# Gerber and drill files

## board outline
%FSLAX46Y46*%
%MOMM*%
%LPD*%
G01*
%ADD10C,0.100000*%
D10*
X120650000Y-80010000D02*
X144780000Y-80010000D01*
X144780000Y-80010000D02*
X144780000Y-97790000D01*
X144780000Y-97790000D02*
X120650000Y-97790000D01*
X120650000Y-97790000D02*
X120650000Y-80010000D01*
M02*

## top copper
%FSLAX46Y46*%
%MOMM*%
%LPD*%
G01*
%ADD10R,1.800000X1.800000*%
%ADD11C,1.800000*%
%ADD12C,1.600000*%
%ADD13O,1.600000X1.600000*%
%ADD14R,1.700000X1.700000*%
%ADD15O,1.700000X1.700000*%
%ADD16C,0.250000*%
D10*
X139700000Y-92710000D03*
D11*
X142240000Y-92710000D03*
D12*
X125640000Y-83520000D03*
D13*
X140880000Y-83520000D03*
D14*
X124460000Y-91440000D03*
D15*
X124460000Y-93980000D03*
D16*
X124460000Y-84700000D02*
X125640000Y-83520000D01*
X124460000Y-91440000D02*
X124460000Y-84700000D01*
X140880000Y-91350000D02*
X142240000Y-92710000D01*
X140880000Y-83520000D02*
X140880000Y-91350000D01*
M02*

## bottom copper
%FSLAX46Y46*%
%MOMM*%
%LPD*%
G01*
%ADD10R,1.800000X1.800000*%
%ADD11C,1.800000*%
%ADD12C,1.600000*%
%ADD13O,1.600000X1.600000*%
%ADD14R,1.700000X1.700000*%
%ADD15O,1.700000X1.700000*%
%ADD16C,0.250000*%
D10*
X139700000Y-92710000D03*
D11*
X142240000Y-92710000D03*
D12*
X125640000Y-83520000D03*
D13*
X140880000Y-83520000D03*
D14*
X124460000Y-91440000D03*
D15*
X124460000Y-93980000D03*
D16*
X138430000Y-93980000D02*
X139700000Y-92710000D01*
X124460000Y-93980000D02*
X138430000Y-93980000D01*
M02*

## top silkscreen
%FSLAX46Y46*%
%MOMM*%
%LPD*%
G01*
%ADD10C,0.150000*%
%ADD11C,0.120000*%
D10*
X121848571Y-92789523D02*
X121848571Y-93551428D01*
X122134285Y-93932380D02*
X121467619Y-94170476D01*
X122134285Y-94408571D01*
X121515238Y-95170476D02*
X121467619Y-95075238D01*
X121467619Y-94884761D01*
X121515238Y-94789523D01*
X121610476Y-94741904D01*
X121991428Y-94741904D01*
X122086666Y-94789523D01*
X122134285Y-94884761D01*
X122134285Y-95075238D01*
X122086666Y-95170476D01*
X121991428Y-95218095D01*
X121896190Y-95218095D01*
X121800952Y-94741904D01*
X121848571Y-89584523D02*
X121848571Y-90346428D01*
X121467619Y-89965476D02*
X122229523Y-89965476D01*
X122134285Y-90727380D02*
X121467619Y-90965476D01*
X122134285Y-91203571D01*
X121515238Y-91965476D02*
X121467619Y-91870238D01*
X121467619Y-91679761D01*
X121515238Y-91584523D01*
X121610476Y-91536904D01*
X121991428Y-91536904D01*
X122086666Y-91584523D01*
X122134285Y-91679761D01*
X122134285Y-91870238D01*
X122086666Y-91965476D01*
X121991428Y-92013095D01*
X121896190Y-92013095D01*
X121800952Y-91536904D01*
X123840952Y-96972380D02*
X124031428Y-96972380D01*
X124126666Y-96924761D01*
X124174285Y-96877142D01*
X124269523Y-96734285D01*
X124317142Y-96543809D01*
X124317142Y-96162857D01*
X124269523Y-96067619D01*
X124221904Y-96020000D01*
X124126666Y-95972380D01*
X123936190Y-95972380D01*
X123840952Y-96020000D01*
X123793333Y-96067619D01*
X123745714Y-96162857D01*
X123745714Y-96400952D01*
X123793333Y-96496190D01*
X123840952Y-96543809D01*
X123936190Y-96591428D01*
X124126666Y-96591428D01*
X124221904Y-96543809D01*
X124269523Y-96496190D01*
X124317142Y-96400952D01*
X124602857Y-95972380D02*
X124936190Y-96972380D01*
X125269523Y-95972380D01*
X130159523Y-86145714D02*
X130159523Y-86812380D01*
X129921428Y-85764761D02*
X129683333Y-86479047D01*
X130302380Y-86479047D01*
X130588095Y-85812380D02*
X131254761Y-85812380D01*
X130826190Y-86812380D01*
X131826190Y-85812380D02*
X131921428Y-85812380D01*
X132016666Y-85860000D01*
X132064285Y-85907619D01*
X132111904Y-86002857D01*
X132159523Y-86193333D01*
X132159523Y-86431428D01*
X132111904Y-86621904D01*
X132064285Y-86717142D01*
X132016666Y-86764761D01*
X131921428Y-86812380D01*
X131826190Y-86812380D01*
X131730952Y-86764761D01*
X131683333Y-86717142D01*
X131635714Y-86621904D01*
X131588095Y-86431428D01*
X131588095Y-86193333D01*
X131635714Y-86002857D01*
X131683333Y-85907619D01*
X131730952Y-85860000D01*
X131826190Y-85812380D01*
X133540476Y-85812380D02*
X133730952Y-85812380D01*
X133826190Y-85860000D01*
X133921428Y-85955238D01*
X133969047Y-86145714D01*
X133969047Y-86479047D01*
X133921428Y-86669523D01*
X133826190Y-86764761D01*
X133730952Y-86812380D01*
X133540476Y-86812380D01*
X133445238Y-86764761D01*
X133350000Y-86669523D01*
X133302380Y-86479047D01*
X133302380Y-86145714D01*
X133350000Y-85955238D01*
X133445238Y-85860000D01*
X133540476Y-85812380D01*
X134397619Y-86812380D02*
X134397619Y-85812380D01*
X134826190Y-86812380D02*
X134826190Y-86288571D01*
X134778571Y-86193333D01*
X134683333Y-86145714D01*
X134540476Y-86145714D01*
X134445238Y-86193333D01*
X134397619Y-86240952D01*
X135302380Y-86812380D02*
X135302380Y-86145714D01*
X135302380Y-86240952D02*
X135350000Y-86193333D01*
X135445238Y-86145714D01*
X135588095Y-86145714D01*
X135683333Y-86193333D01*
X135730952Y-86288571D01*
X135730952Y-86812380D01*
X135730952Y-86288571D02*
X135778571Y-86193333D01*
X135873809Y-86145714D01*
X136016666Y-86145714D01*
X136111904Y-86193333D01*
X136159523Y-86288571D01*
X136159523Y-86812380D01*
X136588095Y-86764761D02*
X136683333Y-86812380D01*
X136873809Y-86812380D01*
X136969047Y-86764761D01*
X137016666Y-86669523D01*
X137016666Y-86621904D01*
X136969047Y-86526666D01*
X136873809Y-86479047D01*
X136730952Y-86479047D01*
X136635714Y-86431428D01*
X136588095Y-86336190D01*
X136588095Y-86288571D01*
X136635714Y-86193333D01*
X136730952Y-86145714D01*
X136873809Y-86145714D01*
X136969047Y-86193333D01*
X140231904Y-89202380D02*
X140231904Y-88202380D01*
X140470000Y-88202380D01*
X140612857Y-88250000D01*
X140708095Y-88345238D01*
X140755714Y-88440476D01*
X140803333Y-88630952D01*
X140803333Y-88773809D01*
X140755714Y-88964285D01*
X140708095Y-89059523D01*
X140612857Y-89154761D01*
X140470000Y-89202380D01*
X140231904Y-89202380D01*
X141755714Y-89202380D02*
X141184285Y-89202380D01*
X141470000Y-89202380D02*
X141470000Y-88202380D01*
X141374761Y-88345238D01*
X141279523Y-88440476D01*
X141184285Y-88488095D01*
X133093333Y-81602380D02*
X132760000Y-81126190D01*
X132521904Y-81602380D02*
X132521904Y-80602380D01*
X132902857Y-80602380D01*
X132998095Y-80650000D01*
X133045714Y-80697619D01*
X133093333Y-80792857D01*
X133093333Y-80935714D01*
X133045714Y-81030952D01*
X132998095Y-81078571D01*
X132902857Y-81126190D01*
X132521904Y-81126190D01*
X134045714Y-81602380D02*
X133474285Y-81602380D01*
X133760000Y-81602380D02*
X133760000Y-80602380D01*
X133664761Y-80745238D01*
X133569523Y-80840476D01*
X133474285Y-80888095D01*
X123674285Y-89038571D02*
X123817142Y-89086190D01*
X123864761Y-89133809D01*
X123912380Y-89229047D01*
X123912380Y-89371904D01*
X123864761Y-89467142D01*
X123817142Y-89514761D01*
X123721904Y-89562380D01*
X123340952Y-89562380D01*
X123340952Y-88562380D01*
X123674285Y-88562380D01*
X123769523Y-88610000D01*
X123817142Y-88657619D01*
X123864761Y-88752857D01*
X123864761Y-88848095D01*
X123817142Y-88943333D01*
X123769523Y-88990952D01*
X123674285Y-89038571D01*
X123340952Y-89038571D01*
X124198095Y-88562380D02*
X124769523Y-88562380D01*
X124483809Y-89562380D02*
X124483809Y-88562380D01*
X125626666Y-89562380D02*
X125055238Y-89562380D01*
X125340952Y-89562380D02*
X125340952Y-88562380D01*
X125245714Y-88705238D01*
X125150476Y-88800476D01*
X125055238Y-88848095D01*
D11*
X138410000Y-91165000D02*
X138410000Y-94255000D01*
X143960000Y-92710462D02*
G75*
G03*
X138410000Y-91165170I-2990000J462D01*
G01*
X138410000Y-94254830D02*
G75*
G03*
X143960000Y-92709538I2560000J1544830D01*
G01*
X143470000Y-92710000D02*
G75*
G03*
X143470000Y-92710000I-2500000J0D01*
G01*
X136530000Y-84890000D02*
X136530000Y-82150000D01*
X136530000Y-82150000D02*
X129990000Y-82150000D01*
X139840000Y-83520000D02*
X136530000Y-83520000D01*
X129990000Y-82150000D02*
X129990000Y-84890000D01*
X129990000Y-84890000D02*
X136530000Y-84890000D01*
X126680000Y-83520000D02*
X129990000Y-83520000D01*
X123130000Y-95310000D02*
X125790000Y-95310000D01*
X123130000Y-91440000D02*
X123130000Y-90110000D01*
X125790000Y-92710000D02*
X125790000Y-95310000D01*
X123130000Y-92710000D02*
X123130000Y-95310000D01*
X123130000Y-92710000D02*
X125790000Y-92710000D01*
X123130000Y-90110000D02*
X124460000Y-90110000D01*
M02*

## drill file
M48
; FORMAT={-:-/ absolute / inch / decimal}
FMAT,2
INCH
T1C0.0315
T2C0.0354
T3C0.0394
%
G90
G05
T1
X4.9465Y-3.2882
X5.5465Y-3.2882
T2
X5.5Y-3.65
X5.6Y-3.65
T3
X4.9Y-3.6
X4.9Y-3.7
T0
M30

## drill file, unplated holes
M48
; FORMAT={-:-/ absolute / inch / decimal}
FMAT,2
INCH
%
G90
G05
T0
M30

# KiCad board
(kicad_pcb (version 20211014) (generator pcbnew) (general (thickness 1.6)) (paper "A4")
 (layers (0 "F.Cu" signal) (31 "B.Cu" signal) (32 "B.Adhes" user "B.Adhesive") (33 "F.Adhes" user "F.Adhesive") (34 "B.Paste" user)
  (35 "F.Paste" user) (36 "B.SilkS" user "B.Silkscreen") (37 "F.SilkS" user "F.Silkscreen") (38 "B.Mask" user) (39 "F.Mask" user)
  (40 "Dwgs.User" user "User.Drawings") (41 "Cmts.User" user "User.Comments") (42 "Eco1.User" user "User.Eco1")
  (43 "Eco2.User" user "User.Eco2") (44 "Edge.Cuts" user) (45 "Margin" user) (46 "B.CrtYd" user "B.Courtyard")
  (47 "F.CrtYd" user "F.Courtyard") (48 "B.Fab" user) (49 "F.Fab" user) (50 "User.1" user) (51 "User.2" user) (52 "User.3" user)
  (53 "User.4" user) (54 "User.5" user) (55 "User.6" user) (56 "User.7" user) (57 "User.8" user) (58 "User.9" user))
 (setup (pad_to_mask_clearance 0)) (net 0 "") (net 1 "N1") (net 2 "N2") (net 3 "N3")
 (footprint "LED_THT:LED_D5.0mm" (layer "F.Cu") (at 139.7 92.71)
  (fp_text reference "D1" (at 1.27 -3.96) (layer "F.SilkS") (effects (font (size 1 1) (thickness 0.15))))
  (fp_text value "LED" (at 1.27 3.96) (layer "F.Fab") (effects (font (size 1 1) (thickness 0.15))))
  (fp_line (start -1.29 -1.545) (end -1.29 1.545) (layer "F.SilkS") (width 0.12))
  (fp_arc (start -1.29 -1.54483) (mid 2.072002 -2.880433) (end 4.26 0.000462) (layer "F.SilkS") (width 0.12))
  (fp_arc (start 4.26 -0.000462) (mid 2.072002 2.880433) (end -1.29 1.54483) (layer "F.SilkS") (width 0.12))
  (fp_circle (center 1.27 0) (end 3.77 0) (layer "F.SilkS") (width 0.12) (fill none))
  (pad "1" thru_hole rect (at 0 0) (size 1.8 1.8) (drill 0.9) (layers *.Cu *.Mask) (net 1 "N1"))
  (pad "2" thru_hole circle (at 2.54 0) (size 1.8 1.8) (drill 0.9) (layers *.Cu *.Mask) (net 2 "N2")))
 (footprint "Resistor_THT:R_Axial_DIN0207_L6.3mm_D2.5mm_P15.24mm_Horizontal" (layer "F.Cu") (at 125.64 83.52)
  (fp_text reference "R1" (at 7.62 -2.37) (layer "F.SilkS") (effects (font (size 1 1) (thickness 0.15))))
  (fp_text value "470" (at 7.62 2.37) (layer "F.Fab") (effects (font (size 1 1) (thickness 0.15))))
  (fp_line (start 10.89 1.37) (end 10.89 -1.37) (layer "F.SilkS") (width 0.12))
  (fp_line (start 10.89 -1.37) (end 4.35 -1.37) (layer "F.SilkS") (width 0.12))
  (fp_line (start 14.2 0) (end 10.89 0) (layer "F.SilkS") (width 0.12))
  (fp_line (start 4.35 -1.37) (end 4.35 1.37) (layer "F.SilkS") (width 0.12))
  (fp_line (start 4.35 1.37) (end 10.89 1.37) (layer "F.SilkS") (width 0.12))
  (fp_line (start 1.04 0) (end 4.35 0) (layer "F.SilkS") (width 0.12))
  (pad "1" thru_hole circle (at 0 0) (size 1.6 1.6) (drill 0.8) (layers *.Cu *.Mask) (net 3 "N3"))
  (pad "2" thru_hole oval (at 15.24 0) (size 1.6 1.6) (drill 0.8) (layers *.Cu *.Mask) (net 2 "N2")))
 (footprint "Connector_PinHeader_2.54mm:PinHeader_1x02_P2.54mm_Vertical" (layer "F.Cu") (at 124.46 91.44)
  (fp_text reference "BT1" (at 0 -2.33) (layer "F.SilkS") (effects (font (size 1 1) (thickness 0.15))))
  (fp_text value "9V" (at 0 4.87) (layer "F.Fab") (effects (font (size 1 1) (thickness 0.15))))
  (fp_line (start -1.33 3.87) (end 1.33 3.87) (layer "F.SilkS") (width 0.12))
  (fp_line (start -1.33 0) (end -1.33 -1.33) (layer "F.SilkS") (width 0.12))
  (fp_line (start 1.33 1.27) (end 1.33 3.87) (layer "F.SilkS") (width 0.12))
  (fp_line (start -1.33 1.27) (end -1.33 3.87) (layer "F.SilkS") (width 0.12))
  (fp_line (start -1.33 1.27) (end 1.33 1.27) (layer "F.SilkS") (width 0.12))
  (fp_line (start -1.33 -1.33) (end 0 -1.33) (layer "F.SilkS") (width 0.12))
  (pad "1" thru_hole rect (at 0 0) (size 1.7 1.7) (drill 1) (layers *.Cu *.Mask) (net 3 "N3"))
  (pad "2" thru_hole oval (at 0 2.54) (size 1.7 1.7) (drill 1) (layers *.Cu *.Mask) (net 1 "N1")))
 (gr_rect (start 120.65 80.01) (end 144.78 97.79) (layer "Edge.Cuts") (width 0.1) (fill none))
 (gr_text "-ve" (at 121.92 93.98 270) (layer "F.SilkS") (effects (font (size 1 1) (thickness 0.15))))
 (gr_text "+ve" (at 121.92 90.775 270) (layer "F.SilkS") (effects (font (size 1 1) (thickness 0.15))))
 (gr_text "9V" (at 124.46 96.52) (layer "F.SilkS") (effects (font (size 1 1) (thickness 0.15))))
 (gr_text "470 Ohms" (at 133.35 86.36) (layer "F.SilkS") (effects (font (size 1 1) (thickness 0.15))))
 (segment (start 124.46 84.7) (end 125.64 83.52) (width 0.25) (layer "F.Cu") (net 3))
 (segment (start 124.46 91.44) (end 124.46 84.7) (width 0.25) (layer "F.Cu") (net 3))
 (segment (start 138.43 93.98) (end 139.7 92.71) (width 0.25) (layer "B.Cu") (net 1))
 (segment (start 124.46 93.98) (end 138.43 93.98) (width 0.25) (layer "B.Cu") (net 1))
 (segment (start 140.88 91.35) (end 142.24 92.71) (width 0.25) (layer "F.Cu") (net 2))
 (segment (start 140.88 83.52) (end 140.88 91.35) (width 0.25) (layer "F.Cu") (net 2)))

